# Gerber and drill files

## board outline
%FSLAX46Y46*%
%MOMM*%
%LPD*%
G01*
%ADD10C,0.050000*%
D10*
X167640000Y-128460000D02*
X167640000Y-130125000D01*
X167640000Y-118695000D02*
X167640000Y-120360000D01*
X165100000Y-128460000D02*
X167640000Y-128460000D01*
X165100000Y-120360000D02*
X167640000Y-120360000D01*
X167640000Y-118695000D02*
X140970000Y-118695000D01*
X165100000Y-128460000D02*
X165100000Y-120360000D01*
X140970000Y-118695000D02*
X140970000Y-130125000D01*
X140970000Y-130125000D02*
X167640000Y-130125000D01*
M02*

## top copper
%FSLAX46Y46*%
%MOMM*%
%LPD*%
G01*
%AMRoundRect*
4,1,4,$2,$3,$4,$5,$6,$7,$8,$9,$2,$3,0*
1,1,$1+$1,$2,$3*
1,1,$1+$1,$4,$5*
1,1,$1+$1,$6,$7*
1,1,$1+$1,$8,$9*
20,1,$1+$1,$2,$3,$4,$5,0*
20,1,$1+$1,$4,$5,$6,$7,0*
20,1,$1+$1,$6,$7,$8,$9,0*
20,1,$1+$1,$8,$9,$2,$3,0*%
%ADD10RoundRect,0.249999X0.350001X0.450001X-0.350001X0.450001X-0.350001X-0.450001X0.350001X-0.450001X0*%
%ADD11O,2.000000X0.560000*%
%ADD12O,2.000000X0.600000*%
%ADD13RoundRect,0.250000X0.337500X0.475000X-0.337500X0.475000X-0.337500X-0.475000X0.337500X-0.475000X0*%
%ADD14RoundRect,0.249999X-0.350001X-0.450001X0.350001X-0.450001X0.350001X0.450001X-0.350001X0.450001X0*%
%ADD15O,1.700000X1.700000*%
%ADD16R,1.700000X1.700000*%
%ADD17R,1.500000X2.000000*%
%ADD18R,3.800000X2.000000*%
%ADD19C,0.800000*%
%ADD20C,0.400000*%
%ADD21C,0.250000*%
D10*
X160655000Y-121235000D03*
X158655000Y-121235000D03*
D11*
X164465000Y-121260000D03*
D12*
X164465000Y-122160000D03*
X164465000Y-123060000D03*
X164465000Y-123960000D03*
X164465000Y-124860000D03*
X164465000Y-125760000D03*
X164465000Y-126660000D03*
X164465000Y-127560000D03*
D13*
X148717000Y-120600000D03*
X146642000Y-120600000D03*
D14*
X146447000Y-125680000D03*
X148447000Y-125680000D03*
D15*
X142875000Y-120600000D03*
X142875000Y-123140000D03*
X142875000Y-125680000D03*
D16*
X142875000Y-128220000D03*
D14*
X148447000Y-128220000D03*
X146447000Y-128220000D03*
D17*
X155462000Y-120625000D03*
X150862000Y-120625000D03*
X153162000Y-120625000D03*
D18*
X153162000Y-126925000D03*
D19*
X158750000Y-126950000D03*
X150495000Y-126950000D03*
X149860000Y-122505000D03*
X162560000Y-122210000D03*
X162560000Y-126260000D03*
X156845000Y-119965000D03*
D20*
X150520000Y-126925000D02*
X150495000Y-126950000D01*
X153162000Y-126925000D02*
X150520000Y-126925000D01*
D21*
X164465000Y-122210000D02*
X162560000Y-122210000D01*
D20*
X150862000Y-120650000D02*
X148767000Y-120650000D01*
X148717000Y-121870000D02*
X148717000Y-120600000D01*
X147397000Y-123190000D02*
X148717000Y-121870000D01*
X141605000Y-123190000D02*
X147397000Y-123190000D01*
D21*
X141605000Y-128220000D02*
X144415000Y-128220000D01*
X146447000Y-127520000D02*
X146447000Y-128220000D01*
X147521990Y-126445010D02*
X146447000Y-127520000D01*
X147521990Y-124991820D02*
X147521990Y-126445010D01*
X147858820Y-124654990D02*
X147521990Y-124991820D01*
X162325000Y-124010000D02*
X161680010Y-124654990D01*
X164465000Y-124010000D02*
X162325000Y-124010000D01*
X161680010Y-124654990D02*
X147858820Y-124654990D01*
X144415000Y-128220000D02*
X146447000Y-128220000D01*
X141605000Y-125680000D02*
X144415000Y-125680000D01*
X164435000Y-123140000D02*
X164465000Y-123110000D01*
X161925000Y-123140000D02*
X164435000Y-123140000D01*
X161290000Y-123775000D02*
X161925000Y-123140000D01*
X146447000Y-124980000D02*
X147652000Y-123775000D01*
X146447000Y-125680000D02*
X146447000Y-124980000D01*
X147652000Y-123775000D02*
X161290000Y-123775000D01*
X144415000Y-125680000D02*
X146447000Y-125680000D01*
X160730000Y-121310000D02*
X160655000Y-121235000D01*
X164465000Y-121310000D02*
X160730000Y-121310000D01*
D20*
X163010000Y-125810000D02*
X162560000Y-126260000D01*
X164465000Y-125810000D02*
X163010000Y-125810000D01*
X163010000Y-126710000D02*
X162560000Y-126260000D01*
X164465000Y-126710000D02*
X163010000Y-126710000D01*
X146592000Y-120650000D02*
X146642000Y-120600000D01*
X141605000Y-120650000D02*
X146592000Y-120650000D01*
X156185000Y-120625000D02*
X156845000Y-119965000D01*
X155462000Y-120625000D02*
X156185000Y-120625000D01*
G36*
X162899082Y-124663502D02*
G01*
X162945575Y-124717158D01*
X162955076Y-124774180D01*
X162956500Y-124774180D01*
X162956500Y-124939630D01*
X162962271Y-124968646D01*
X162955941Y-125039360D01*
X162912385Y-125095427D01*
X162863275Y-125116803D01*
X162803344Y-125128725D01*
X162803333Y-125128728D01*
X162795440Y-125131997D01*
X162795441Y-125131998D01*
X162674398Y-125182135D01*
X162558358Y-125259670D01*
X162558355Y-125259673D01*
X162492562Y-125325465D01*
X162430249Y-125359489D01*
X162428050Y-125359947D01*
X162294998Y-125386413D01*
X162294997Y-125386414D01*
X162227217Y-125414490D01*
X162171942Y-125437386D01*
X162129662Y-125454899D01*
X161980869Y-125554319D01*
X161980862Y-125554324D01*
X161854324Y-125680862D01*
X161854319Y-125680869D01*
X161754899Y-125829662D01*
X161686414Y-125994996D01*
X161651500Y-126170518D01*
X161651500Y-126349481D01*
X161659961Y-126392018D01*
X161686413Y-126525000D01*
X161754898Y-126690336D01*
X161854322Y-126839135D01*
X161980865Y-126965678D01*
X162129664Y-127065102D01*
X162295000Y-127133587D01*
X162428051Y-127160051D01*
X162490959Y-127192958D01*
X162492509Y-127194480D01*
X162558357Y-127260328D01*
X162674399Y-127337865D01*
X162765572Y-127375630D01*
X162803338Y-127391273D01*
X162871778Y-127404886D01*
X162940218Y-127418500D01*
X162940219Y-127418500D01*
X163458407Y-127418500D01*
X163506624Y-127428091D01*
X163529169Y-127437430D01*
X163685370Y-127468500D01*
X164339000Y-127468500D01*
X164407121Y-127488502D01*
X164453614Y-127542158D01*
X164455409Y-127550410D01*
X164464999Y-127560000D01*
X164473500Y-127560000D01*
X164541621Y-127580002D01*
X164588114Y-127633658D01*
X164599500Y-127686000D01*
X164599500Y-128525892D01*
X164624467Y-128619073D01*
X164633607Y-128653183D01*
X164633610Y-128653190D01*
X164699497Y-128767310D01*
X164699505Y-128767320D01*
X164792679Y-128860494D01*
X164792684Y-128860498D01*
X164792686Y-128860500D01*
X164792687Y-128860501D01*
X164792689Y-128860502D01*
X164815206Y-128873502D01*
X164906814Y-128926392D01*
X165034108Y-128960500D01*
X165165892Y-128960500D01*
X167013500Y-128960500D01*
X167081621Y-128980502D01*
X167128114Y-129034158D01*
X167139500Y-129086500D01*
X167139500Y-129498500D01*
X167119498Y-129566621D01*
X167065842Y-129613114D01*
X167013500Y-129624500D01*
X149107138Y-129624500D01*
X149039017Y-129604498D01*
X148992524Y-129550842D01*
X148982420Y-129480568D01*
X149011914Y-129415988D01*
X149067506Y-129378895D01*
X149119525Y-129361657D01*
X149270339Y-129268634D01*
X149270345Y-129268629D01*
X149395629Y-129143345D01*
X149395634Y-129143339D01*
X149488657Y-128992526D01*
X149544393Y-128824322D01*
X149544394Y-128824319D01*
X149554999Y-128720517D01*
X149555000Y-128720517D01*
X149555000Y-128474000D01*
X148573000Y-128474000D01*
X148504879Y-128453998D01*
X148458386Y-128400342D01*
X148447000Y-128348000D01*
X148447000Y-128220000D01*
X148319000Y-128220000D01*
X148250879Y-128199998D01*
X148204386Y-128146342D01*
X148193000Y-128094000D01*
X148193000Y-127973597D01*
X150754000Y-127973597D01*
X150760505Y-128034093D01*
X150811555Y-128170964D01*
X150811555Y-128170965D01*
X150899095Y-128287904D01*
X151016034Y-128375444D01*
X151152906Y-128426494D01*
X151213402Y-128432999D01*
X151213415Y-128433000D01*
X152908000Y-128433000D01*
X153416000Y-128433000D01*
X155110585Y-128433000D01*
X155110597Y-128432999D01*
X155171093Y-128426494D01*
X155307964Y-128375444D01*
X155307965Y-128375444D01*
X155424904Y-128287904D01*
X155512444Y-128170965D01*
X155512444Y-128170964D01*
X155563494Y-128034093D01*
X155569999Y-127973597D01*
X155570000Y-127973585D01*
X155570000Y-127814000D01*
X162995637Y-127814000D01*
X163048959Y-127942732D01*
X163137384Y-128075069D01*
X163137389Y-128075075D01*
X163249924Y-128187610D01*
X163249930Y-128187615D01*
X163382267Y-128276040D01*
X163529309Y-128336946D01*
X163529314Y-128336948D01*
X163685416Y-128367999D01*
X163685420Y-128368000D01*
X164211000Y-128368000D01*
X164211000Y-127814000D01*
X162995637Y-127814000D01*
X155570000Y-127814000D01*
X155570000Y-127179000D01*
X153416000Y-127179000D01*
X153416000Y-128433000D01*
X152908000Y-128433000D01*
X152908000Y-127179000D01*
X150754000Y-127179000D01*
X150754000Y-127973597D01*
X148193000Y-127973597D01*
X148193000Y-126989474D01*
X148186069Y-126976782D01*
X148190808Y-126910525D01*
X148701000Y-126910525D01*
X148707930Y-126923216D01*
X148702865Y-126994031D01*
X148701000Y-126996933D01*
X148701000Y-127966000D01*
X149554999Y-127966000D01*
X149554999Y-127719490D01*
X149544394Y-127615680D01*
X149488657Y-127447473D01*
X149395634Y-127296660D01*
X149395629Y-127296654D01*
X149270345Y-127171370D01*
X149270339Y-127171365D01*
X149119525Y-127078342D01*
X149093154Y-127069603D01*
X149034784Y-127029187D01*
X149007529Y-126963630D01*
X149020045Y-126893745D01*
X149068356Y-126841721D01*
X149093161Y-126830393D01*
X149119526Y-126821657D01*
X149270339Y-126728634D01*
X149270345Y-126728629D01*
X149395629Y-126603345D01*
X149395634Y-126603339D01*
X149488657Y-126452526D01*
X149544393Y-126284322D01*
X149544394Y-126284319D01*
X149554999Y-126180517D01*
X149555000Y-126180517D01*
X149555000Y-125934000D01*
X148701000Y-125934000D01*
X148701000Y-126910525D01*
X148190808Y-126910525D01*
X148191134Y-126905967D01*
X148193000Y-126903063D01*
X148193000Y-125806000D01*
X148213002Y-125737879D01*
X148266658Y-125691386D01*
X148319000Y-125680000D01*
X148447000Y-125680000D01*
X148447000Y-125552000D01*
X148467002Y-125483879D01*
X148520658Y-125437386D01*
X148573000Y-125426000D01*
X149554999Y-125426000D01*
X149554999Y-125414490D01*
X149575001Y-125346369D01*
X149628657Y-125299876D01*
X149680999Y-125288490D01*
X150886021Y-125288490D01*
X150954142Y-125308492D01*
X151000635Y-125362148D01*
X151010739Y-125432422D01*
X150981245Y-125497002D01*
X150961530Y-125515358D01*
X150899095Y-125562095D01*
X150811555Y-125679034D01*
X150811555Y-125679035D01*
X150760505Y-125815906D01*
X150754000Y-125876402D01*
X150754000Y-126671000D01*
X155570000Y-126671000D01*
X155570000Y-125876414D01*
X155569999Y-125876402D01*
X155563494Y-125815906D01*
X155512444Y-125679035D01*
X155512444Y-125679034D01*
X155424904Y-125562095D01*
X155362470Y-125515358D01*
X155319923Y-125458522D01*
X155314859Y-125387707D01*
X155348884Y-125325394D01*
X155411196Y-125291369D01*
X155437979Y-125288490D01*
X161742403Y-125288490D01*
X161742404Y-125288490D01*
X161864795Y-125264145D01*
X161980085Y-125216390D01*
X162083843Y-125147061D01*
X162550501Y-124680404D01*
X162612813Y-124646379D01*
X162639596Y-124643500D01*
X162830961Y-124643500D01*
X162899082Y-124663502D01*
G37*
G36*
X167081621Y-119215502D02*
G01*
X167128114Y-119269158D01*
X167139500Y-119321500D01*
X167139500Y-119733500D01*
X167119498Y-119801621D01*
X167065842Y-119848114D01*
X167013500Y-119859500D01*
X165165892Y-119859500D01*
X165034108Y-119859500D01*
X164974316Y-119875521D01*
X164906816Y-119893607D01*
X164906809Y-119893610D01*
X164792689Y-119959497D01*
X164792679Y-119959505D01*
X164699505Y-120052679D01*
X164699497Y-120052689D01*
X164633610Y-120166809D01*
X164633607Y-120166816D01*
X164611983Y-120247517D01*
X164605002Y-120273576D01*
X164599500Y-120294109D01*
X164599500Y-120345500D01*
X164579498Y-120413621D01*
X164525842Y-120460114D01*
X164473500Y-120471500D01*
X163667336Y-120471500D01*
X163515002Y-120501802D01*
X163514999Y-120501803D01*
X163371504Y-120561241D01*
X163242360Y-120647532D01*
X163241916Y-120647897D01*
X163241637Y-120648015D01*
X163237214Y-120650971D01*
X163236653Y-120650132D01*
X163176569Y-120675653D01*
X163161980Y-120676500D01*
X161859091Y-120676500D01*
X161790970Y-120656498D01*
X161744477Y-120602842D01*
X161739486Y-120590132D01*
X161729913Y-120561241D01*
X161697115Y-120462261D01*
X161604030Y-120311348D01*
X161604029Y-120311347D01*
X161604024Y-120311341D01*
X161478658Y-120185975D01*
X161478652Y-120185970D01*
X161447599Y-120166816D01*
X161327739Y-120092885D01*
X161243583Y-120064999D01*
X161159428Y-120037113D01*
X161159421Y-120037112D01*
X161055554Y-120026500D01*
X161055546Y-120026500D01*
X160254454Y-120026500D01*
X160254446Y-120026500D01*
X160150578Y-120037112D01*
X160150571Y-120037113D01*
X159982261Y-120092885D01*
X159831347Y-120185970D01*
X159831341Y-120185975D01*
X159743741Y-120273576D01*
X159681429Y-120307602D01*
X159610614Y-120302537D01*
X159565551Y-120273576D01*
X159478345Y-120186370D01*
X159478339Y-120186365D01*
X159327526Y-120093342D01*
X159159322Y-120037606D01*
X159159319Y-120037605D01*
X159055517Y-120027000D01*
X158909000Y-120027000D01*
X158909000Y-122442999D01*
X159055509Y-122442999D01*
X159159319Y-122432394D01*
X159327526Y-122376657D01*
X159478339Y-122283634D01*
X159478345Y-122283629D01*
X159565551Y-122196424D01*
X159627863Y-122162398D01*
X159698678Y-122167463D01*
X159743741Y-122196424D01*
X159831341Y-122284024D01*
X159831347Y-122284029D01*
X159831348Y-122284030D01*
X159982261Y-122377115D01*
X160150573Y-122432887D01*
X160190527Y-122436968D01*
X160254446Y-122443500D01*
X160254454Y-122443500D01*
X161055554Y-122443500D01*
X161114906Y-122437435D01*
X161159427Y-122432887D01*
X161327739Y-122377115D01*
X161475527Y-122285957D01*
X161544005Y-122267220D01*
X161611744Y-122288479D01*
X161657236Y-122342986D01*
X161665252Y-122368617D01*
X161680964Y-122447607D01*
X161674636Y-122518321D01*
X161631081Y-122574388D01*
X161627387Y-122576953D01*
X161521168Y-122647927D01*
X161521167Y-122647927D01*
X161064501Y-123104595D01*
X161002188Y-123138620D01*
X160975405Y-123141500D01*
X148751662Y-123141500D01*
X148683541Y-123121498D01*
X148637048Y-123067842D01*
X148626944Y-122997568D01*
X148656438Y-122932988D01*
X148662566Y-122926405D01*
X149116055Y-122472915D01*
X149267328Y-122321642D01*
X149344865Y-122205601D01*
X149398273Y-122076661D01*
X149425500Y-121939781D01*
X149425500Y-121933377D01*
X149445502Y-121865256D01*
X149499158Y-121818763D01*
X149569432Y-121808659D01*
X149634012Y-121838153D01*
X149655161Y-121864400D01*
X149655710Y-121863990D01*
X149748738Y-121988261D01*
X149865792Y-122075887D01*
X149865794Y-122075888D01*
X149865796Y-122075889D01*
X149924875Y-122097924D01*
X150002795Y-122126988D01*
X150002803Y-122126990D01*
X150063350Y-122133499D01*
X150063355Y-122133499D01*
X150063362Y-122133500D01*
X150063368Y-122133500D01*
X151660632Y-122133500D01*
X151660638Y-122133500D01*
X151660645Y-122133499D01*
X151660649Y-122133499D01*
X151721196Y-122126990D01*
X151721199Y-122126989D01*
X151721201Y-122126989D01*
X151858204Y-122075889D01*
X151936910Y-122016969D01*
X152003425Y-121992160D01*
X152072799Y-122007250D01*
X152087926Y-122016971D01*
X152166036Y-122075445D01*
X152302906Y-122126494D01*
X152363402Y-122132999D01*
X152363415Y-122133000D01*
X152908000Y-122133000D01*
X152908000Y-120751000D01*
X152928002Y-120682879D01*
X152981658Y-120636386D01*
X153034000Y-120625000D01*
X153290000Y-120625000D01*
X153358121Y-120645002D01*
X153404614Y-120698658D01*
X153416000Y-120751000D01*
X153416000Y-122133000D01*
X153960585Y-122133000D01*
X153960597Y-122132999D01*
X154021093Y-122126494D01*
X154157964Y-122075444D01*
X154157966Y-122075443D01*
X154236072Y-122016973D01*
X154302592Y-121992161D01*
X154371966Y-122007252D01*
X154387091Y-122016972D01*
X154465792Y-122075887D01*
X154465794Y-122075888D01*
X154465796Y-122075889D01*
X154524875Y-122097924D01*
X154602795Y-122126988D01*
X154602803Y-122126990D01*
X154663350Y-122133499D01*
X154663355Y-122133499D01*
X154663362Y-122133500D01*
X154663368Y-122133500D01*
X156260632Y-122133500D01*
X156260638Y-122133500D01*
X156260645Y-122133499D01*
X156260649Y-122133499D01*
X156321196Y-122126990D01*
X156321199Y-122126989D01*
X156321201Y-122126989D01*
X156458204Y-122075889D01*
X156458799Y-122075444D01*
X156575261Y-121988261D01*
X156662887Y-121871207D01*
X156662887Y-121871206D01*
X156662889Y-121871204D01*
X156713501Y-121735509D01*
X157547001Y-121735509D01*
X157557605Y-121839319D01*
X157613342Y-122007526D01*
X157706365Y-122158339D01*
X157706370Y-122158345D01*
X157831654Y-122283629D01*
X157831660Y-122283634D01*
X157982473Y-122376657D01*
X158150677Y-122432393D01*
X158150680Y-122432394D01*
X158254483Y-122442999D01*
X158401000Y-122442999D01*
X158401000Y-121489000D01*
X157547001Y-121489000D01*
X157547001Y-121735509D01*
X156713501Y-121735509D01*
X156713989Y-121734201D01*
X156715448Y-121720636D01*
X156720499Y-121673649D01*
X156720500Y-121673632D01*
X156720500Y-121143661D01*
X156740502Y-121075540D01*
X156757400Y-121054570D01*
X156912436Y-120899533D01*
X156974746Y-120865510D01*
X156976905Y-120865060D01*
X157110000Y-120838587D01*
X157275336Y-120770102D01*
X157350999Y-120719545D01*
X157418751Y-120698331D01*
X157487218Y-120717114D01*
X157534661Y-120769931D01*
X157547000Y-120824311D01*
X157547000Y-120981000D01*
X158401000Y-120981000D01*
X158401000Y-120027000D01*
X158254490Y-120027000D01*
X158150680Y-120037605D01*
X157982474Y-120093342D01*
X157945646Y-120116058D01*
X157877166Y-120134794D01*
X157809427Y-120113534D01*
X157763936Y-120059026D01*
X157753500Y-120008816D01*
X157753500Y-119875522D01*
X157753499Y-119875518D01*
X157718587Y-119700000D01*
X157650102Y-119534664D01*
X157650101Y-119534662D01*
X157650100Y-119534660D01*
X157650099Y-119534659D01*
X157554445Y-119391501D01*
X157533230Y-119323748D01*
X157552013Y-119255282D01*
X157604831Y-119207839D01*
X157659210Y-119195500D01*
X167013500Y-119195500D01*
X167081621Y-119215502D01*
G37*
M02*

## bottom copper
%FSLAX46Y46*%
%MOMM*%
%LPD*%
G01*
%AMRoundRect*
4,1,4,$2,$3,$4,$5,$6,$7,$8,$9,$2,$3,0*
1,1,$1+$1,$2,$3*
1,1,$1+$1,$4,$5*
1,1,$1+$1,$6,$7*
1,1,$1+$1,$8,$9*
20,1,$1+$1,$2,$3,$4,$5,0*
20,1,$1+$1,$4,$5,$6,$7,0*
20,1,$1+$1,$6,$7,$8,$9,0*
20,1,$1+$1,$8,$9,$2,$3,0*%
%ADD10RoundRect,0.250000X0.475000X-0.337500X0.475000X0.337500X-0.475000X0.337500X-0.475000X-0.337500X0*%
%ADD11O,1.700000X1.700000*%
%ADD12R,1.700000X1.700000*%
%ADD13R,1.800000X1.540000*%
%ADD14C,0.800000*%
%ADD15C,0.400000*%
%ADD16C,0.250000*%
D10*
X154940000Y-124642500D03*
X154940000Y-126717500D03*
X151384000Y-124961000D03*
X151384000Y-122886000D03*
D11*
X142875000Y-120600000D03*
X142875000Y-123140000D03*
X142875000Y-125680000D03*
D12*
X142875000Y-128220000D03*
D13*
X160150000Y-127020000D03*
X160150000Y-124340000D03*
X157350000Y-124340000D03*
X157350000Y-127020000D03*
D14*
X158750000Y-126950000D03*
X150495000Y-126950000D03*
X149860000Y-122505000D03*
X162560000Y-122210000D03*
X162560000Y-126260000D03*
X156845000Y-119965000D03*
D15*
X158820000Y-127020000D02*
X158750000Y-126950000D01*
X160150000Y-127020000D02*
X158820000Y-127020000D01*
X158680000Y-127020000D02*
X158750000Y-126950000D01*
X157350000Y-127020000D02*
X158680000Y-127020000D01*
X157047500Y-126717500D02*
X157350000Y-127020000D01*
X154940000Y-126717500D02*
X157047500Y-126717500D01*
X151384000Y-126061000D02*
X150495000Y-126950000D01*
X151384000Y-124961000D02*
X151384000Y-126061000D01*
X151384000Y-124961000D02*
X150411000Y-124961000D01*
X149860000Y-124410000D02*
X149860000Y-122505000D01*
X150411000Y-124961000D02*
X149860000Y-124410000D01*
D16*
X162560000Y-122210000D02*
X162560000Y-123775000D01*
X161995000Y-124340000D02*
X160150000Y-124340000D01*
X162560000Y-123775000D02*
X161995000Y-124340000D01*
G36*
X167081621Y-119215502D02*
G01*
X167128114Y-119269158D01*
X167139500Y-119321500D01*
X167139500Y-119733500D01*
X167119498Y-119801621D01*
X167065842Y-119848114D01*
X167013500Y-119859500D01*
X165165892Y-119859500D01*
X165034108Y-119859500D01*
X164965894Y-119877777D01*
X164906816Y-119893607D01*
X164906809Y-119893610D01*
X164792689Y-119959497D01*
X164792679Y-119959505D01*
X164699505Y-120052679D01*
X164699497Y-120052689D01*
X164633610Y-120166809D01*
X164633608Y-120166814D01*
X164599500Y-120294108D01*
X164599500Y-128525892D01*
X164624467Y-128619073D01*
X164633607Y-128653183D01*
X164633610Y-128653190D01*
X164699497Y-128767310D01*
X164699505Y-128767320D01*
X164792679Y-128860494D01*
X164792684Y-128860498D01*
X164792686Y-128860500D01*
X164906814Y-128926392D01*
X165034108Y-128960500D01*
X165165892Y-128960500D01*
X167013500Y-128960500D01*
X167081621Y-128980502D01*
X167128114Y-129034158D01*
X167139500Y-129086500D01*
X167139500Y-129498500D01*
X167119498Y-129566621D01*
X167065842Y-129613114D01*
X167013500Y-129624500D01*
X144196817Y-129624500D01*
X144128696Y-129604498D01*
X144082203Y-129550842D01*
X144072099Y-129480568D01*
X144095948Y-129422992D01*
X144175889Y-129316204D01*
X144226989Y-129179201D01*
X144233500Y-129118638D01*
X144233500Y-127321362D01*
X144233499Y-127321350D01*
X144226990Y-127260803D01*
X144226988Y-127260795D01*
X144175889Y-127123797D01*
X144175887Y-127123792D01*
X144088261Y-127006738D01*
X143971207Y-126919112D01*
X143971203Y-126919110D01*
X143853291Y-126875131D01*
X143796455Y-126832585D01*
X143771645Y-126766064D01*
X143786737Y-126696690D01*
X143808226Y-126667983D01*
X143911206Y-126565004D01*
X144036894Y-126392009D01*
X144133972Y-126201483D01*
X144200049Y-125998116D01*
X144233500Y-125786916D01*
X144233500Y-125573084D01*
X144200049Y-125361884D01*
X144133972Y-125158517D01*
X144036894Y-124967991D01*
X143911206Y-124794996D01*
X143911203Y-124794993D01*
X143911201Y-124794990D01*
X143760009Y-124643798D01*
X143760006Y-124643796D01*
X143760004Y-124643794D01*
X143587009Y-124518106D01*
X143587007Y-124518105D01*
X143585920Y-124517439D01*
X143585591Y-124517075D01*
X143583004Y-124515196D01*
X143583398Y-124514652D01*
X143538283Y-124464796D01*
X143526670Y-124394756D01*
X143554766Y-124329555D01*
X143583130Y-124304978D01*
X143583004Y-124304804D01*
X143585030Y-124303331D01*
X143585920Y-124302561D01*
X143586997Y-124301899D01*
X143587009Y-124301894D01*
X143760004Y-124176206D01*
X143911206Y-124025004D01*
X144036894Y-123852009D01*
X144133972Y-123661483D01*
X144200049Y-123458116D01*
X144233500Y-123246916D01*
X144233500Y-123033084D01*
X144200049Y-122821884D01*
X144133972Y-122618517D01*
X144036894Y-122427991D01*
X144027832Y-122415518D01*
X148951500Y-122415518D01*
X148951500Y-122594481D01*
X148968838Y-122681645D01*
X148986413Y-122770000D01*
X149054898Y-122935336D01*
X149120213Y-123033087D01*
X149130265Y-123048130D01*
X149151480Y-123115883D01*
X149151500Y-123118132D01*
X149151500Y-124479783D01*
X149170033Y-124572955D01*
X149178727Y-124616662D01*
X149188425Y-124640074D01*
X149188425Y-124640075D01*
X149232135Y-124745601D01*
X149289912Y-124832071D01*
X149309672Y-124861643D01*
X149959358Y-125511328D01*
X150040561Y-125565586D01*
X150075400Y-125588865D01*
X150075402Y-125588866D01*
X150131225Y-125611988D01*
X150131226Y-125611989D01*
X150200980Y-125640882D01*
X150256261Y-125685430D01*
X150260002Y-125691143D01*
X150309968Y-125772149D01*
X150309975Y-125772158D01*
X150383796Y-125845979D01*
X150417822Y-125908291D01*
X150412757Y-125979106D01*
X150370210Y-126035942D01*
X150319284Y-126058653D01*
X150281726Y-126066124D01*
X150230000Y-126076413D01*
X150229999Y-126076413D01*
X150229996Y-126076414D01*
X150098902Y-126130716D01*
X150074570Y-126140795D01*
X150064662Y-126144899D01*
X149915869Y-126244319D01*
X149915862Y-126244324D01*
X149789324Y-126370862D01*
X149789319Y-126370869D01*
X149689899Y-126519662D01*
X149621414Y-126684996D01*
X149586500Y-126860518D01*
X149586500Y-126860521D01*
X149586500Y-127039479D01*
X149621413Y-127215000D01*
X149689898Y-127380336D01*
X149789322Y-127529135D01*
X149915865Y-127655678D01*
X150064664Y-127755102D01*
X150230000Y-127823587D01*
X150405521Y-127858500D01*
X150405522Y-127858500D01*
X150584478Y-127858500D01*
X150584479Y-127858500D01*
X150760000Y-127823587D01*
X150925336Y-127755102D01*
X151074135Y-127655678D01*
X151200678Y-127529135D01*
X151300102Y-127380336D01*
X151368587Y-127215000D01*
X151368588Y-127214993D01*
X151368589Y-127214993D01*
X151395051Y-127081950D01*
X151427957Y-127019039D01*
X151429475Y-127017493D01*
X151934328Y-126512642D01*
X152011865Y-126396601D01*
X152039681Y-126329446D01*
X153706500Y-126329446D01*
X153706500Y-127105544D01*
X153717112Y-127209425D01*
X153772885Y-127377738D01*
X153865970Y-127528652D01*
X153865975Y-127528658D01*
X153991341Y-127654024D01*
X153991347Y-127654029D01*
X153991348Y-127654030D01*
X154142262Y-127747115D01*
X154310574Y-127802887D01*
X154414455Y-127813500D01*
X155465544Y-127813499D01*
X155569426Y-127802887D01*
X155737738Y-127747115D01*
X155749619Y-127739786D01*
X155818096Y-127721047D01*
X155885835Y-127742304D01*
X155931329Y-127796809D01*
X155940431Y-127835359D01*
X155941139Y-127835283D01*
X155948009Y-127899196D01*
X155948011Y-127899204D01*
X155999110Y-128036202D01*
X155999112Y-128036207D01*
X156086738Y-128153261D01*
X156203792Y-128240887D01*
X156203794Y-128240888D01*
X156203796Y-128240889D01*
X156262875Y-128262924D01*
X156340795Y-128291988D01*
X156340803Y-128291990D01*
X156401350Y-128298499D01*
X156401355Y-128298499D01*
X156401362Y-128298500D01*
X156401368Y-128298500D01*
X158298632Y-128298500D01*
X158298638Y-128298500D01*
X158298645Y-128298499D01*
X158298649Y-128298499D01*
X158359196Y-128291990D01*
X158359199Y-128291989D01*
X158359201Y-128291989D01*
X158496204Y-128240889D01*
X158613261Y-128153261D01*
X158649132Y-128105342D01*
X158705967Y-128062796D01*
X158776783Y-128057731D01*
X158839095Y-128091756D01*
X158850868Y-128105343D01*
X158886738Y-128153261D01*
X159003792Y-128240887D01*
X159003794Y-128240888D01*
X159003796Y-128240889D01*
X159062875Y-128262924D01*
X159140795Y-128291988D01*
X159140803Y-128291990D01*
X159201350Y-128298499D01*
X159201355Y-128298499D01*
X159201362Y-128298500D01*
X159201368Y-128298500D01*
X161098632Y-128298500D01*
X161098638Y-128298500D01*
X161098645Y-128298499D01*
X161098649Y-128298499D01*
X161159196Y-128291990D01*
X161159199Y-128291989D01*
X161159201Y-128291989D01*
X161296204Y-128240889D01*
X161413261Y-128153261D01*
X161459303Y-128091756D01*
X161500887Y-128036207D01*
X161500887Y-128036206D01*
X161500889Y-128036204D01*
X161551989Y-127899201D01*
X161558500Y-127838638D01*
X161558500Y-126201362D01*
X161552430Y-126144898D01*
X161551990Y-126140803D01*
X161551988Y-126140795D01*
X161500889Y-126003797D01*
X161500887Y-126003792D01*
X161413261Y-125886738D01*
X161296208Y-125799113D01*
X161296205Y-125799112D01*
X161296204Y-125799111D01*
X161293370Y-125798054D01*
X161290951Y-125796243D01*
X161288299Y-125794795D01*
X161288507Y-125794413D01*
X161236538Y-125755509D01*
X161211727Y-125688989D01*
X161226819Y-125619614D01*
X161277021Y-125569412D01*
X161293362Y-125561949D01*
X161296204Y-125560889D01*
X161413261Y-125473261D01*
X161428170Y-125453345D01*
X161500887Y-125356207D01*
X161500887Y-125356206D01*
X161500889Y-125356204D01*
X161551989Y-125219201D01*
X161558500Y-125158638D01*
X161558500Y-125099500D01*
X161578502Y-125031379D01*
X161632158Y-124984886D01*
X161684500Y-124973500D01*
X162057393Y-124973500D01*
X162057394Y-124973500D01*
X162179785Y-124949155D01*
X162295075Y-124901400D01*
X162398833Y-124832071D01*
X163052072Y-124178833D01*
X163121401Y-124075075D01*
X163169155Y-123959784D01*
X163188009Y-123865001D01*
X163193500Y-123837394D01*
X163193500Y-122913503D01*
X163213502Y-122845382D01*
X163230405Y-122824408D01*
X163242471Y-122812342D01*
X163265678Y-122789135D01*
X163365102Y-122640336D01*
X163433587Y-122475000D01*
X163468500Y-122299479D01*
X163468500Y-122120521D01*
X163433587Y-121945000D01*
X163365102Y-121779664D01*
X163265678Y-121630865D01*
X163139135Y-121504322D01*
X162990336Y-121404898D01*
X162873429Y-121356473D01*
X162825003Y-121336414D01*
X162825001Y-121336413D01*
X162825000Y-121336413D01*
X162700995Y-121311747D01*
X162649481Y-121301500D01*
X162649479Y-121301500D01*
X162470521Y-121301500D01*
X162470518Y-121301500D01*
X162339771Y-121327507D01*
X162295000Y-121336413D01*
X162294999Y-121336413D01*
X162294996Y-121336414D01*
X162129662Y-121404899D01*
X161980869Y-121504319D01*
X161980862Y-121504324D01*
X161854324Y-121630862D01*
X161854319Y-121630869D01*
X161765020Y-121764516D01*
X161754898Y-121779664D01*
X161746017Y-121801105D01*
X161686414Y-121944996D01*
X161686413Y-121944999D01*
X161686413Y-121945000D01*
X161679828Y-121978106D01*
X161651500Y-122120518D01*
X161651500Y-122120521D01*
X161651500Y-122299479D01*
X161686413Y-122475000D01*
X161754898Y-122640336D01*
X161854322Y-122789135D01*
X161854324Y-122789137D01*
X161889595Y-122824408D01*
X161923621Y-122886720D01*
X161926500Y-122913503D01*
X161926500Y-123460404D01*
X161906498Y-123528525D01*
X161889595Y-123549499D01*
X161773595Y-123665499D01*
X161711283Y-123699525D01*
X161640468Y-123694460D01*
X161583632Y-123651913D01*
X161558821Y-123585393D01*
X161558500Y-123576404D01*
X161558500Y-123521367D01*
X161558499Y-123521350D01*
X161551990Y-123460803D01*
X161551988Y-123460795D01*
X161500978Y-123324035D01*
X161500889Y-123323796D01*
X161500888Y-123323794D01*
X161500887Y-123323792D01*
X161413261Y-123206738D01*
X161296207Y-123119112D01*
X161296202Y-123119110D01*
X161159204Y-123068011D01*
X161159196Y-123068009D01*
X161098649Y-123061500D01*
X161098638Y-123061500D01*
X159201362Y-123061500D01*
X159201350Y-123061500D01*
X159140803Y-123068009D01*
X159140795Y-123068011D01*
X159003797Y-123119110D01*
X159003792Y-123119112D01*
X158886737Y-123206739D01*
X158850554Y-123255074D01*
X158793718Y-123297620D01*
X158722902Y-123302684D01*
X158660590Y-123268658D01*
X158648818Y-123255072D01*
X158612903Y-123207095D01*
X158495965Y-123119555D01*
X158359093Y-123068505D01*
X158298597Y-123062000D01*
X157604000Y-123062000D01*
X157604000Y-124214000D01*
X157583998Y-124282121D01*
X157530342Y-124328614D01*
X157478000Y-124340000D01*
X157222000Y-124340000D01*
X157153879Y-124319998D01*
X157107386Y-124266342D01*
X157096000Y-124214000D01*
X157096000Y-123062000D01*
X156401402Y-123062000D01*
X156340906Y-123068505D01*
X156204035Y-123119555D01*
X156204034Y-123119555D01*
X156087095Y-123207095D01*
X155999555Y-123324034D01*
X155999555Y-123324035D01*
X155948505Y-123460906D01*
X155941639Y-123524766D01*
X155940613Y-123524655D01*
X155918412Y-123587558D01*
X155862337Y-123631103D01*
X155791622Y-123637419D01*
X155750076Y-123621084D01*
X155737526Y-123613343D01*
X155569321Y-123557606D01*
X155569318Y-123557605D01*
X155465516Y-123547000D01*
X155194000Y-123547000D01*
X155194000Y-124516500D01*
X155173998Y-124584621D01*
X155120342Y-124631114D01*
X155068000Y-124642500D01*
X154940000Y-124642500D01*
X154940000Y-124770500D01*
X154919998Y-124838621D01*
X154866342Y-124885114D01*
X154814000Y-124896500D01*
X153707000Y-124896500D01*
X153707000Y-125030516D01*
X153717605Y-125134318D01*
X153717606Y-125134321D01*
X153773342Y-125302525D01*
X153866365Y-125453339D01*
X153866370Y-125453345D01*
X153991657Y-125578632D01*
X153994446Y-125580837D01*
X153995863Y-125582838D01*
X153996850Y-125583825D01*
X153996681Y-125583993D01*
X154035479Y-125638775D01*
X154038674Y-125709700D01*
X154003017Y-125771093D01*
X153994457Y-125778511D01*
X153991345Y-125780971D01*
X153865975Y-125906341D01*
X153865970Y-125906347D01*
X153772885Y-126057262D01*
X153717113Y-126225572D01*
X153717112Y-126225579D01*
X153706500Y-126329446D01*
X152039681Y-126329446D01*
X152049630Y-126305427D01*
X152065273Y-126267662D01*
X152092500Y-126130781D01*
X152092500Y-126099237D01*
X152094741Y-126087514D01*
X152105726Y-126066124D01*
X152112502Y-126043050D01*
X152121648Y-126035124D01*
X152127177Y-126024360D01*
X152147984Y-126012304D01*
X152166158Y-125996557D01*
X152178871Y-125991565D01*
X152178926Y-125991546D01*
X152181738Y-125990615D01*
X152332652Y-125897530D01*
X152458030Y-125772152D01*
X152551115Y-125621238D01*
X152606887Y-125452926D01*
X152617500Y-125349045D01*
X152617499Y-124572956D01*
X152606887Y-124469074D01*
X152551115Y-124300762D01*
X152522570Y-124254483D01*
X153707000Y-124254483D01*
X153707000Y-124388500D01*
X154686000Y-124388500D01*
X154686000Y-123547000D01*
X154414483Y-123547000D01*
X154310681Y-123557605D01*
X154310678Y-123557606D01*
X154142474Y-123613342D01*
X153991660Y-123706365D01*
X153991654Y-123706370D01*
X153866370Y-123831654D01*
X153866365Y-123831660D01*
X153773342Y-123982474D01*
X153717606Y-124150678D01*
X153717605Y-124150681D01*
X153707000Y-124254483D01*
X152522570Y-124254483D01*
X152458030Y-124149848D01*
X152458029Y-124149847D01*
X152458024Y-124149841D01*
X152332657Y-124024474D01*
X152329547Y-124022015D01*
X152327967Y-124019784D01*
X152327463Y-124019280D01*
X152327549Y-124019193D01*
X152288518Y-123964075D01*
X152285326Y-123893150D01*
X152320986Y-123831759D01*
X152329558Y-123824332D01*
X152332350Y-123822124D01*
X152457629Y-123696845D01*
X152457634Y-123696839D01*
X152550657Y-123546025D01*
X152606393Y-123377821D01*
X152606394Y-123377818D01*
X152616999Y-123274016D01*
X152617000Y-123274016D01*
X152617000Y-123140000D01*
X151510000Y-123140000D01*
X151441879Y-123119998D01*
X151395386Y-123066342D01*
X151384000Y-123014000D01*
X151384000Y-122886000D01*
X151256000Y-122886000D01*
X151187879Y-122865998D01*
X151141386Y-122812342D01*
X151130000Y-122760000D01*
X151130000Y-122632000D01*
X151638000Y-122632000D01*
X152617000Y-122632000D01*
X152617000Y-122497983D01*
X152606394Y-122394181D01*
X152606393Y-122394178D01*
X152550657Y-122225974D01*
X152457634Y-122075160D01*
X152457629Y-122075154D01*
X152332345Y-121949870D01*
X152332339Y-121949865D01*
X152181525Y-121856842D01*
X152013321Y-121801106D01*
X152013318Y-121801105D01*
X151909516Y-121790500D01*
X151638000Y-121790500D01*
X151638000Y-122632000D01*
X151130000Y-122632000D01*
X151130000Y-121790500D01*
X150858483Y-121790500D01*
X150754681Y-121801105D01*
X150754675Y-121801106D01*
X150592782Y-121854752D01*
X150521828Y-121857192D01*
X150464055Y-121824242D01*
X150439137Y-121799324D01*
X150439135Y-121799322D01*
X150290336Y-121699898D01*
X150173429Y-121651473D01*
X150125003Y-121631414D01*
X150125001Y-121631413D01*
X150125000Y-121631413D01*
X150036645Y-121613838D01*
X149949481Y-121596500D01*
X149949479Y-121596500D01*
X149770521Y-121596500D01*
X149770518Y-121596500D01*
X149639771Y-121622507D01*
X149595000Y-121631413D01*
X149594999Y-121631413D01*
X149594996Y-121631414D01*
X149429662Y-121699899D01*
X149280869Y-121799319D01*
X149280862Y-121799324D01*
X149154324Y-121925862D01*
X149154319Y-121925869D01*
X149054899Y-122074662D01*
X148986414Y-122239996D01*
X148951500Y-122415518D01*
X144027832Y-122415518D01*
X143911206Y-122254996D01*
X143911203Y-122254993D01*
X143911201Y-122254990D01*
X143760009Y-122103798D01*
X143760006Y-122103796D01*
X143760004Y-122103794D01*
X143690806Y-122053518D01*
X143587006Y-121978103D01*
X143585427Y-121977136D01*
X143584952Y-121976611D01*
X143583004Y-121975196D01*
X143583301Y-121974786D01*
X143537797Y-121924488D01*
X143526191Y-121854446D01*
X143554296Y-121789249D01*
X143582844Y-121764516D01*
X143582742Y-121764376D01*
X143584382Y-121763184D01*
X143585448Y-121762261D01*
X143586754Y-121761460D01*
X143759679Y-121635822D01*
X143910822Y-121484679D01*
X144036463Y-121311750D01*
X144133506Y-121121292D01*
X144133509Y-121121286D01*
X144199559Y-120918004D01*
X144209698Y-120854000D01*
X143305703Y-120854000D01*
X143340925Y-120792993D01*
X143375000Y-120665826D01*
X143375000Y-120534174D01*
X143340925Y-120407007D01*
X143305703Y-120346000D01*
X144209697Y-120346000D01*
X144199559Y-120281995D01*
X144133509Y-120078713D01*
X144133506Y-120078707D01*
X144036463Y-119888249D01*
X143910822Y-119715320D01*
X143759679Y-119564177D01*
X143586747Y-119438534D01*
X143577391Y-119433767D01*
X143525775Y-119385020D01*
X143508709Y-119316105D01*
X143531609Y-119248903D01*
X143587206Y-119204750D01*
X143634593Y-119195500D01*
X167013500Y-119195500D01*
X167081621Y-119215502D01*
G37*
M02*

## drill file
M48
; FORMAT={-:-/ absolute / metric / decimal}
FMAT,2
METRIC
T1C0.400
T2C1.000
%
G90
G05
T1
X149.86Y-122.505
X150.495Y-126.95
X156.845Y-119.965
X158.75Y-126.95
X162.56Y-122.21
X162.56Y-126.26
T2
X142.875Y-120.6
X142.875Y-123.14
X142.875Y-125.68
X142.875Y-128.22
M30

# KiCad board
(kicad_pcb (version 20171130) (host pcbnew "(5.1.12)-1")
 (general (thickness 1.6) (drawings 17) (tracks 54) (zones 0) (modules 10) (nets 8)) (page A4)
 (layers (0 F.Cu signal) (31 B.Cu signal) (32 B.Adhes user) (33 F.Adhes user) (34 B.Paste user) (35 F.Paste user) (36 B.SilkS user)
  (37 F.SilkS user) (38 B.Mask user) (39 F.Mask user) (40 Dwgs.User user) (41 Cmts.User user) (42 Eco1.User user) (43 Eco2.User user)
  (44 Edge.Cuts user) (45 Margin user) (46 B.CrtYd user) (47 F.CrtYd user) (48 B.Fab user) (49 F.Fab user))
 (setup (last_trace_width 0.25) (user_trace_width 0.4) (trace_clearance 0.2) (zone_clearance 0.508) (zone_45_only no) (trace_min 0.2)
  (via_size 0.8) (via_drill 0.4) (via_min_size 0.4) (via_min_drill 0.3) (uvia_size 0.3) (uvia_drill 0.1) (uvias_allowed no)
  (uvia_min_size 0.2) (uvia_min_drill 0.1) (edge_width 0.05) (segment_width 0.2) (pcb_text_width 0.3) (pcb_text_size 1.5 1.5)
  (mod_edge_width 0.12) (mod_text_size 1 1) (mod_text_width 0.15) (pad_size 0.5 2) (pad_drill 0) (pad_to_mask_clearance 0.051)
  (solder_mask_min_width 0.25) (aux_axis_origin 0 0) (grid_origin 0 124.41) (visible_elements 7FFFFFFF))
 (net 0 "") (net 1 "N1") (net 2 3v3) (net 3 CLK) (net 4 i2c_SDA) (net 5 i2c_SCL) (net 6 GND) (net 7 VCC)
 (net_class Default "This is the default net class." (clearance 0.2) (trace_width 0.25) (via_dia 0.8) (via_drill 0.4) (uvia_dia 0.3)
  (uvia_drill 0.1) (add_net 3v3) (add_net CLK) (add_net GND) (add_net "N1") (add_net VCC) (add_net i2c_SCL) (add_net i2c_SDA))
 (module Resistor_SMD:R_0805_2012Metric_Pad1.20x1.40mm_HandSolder (layer F.Cu) (at 159.655 121.235 180)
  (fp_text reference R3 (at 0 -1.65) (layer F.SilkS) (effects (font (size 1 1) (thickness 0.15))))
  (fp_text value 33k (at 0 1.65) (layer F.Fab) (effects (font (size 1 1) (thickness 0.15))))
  (pad 1 smd roundrect (at -1 0 180) (size 1.2 1.4) (layers F.Cu F.Paste F.Mask) (roundrect_rratio 0.2083325) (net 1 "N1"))
  (pad 2 smd roundrect (at 1 0 180) (size 1.2 1.4) (layers F.Cu F.Paste F.Mask) (roundrect_rratio 0.2083325) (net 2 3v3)))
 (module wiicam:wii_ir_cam (layer F.Cu) (at 164.465 124.41 90)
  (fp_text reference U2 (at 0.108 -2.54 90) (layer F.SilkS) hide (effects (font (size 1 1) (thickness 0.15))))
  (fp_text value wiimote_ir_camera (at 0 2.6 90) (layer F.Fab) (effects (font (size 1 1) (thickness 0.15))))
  (pad 8 smd oval (at 3.15 0 90) (size 0.56 2) (layers F.Cu F.Paste F.Mask) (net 1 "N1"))
  (pad 7 smd oval (at 2.25 0 90) (size 0.6 2) (layers F.Cu F.Paste F.Mask) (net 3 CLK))
  (pad 6 smd oval (at 1.35 0 90) (size 0.6 2) (layers F.Cu F.Paste F.Mask) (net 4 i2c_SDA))
  (pad 5 smd oval (at 0.45 0 90) (size 0.6 2) (layers F.Cu F.Paste F.Mask) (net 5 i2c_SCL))
  (pad 4 smd oval (at -0.45 0 90) (size 0.6 2) (layers F.Cu F.Paste F.Mask))
  (pad 3 smd oval (at -1.35 0 90) (size 0.6 2) (layers F.Cu F.Paste F.Mask) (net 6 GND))
  (pad 2 smd oval (at -2.25 0 90) (size 0.6 2) (layers F.Cu F.Paste F.Mask) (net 6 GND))
  (pad 1 smd oval (at -3.15 0 90) (size 0.6 2) (layers F.Cu F.Paste F.Mask) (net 2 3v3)))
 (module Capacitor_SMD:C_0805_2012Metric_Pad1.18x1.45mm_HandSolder (layer B.Cu) (at 154.94 125.68 90)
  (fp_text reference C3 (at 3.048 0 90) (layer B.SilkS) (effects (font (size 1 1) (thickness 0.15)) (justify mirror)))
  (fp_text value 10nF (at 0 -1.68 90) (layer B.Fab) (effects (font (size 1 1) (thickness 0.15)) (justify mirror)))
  (pad 2 smd roundrect (at 1.0375 0 90) (size 1.175 1.45) (layers B.Cu B.Paste B.Mask) (roundrect_rratio 0.2127659574468085) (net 6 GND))
  (pad 1 smd roundrect (at -1.0375 0 90) (size 1.175 1.45) (layers B.Cu B.Paste B.Mask) (roundrect_rratio 0.2127659574468085) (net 2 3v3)))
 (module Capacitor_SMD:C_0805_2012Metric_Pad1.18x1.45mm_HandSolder (layer F.Cu) (at 147.6795 120.6 180)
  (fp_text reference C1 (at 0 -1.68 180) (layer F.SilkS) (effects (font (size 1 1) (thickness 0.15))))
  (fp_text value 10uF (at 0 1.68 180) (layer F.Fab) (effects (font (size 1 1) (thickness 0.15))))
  (pad 1 smd roundrect (at -1.0375 0 180) (size 1.175 1.45) (layers F.Cu F.Paste F.Mask) (roundrect_rratio 0.2127659574468085) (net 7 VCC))
  (pad 2 smd roundrect (at 1.0375 0 180) (size 1.175 1.45) (layers F.Cu F.Paste F.Mask) (roundrect_rratio 0.2127659574468085) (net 6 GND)))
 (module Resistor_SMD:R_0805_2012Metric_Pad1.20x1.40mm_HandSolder (layer F.Cu) (at 147.447 125.68)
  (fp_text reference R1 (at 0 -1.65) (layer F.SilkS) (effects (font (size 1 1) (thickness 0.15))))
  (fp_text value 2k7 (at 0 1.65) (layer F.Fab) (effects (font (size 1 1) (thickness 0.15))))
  (pad 1 smd roundrect (at -1 0) (size 1.2 1.4) (layers F.Cu F.Paste F.Mask) (roundrect_rratio 0.2083325) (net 4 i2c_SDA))
  (pad 2 smd roundrect (at 1 0) (size 1.2 1.4) (layers F.Cu F.Paste F.Mask) (roundrect_rratio 0.2083325) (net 2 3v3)))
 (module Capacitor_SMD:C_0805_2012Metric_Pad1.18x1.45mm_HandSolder (layer B.Cu) (at 151.384 123.9235 90)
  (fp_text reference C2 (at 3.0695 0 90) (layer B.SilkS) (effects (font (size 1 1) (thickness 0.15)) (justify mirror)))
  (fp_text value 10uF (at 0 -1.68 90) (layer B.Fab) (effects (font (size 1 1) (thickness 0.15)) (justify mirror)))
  (pad 1 smd roundrect (at -1.0375 0 90) (size 1.175 1.45) (layers B.Cu B.Paste B.Mask) (roundrect_rratio 0.2127659574468085) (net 2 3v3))
  (pad 2 smd roundrect (at 1.0375 0 90) (size 1.175 1.45) (layers B.Cu B.Paste B.Mask) (roundrect_rratio 0.2127659574468085) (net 6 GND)))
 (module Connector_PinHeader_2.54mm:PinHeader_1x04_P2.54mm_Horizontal (layer F.Cu) (at 142.875 128.22 180)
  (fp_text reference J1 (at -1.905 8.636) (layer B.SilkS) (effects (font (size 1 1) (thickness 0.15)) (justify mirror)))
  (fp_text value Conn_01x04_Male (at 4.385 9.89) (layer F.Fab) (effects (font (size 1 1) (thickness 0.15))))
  (pad 4 thru_hole oval (at 0 7.62 180) (size 1.7 1.7) (drill 1) (layers *.Cu *.Mask) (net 6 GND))
  (pad 3 thru_hole oval (at 0 5.08 180) (size 1.7 1.7) (drill 1) (layers *.Cu *.Mask) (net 7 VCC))
  (pad 2 thru_hole oval (at 0 2.54 180) (size 1.7 1.7) (drill 1) (layers *.Cu *.Mask) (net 4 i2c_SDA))
  (pad 1 thru_hole rect (at 0 0 180) (size 1.7 1.7) (drill 1) (layers *.Cu *.Mask) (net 5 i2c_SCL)))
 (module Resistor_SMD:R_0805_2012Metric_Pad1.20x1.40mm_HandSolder (layer F.Cu) (at 147.447 128.22)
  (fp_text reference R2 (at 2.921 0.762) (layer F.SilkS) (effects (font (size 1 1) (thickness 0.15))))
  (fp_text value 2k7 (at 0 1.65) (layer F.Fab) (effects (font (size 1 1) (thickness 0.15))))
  (pad 2 smd roundrect (at 1 0) (size 1.2 1.4) (layers F.Cu F.Paste F.Mask) (roundrect_rratio 0.2083325) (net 2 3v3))
  (pad 1 smd roundrect (at -1 0) (size 1.2 1.4) (layers F.Cu F.Paste F.Mask) (roundrect_rratio 0.2083325) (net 5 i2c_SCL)))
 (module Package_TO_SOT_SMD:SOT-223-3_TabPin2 (layer F.Cu) (at 153.162 123.775 270)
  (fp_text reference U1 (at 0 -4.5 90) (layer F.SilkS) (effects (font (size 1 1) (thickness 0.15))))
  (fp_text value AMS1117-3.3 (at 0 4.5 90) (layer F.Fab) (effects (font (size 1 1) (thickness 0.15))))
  (pad 1 smd rect (at -3.15 -2.3 270) (size 2 1.5) (layers F.Cu F.Paste F.Mask) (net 6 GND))
  (pad 3 smd rect (at -3.15 2.3 270) (size 2 1.5) (layers F.Cu F.Paste F.Mask) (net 7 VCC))
  (pad 2 smd rect (at -3.15 0 270) (size 2 1.5) (layers F.Cu F.Paste F.Mask) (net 2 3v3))
  (pad 2 smd rect (at 3.15 0 270) (size 2 3.8) (layers F.Cu F.Paste F.Mask) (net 2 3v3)))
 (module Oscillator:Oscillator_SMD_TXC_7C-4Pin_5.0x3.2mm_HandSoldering (layer B.Cu) (at 158.75 125.68 90)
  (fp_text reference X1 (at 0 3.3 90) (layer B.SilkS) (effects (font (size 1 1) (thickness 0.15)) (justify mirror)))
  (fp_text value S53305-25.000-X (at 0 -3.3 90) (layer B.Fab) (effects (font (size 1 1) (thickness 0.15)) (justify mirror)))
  (pad 4 smd rect (at -1.34 1.4 90) (size 1.54 1.8) (layers B.Cu B.Paste B.Mask) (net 2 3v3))
  (pad 3 smd rect (at 1.34 1.4 90) (size 1.54 1.8) (layers B.Cu B.Paste B.Mask) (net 3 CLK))
  (pad 2 smd rect (at 1.34 -1.4 90) (size 1.54 1.8) (layers B.Cu B.Paste B.Mask) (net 6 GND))
  (pad 1 smd rect (at -1.34 -1.4 90) (size 1.54 1.8) (layers B.Cu B.Paste B.Mask) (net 2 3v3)))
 (gr_line (start 167.64 128.46) (end 167.64 130.125) (layer Edge.Cuts) (width 0.05))
 (gr_line (start 167.64 118.695) (end 167.64 120.36) (layer Edge.Cuts) (width 0.05))
 (gr_line (start 165.1 128.46) (end 167.64 128.46) (layer Edge.Cuts) (width 0.05))
 (gr_line (start 165.1 120.36) (end 167.64 120.36) (layer Edge.Cuts) (width 0.05))
 (gr_line (start 167.64 118.695) (end 140.97 118.695) (layer Edge.Cuts) (width 0.05))
 (gr_line (start 165.1 128.46) (end 165.1 120.36) (layer Edge.Cuts) (width 0.05))
 (gr_line (start 140.97 118.695) (end 140.97 130.125) (layer Edge.Cuts) (width 0.05))
 (gr_line (start 140.97 130.125) (end 167.64 130.125) (layer Edge.Cuts) (width 0.05))
 (via (at 158.75 126.95) (size 0.8) (drill 0.4) (layers F.Cu B.Cu) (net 2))
 (segment (start 158.82 127.02) (end 158.75 126.95) (width 0.4) (layer B.Cu) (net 2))
 (segment (start 160.15 127.02) (end 158.82 127.02) (width 0.4) (layer B.Cu) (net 2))
 (segment (start 158.68 127.02) (end 158.75 126.95) (width 0.4) (layer B.Cu) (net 2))
 (segment (start 157.35 127.02) (end 158.68 127.02) (width 0.4) (layer B.Cu) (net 2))
 (segment (start 157.0475 126.7175) (end 157.35 127.02) (width 0.4) (layer B.Cu) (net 2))
 (segment (start 154.94 126.7175) (end 157.0475 126.7175) (width 0.4) (layer B.Cu) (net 2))
 (via (at 150.495 126.95) (size 0.8) (drill 0.4) (layers F.Cu B.Cu) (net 2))
 (segment (start 150.52 126.925) (end 150.495 126.95) (width 0.4) (layer F.Cu) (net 2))
 (segment (start 153.162 126.925) (end 150.52 126.925) (width 0.4) (layer F.Cu) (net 2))
 (segment (start 151.384 126.061) (end 150.495 126.95) (width 0.4) (layer B.Cu) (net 2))
 (segment (start 151.384 124.961) (end 151.384 126.061) (width 0.4) (layer B.Cu) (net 2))
 (segment (start 151.384 124.961) (end 150.411 124.961) (width 0.4) (layer B.Cu) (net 2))
 (via (at 149.86 122.505) (size 0.8) (drill 0.4) (layers F.Cu B.Cu) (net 2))
 (segment (start 149.86 124.41) (end 149.86 122.505) (width 0.4) (layer B.Cu) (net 2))
 (segment (start 150.411 124.961) (end 149.86 124.41) (width 0.4) (layer B.Cu) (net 2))
 (via (at 162.56 122.21) (size 0.8) (drill 0.4) (layers F.Cu B.Cu) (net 3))
 (segment (start 164.465 122.21) (end 162.56 122.21) (width 0.25) (layer F.Cu) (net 3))
 (segment (start 162.56 122.21) (end 162.56 123.775) (width 0.25) (layer B.Cu) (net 3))
 (segment (start 161.995 124.34) (end 160.15 124.34) (width 0.25) (layer B.Cu) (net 3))
 (segment (start 162.56 123.775) (end 161.995 124.34) (width 0.25) (layer B.Cu) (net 3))
 (segment (start 150.862 120.65) (end 148.767 120.65) (width 0.4) (layer F.Cu) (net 7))
 (segment (start 148.717 121.87) (end 148.717 120.6) (width 0.4) (layer F.Cu) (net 7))
 (segment (start 147.397 123.19) (end 148.717 121.87) (width 0.4) (layer F.Cu) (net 7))
 (segment (start 141.605 123.19) (end 147.397 123.19) (width 0.4) (layer F.Cu) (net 7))
 (segment (start 141.605 128.22) (end 144.415 128.22) (width 0.25) (layer F.Cu) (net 5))
 (segment (start 146.447 127.52) (end 146.447 128.22) (width 0.25) (layer F.Cu) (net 5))
 (segment (start 147.52199 126.44501) (end 146.447 127.52) (width 0.25) (layer F.Cu) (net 5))
 (segment (start 147.52199 124.99182) (end 147.52199 126.44501) (width 0.25) (layer F.Cu) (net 5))
 (segment (start 147.85882 124.65499) (end 147.52199 124.99182) (width 0.25) (layer F.Cu) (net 5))
 (segment (start 162.325 124.01) (end 161.68001 124.65499) (width 0.25) (layer F.Cu) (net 5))
 (segment (start 164.465 124.01) (end 162.325 124.01) (width 0.25) (layer F.Cu) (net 5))
 (segment (start 161.68001 124.65499) (end 147.85882 124.65499) (width 0.25) (layer F.Cu) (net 5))
 (segment (start 144.415 128.22) (end 146.447 128.22) (width 0.25) (layer F.Cu) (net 5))
 (segment (start 141.605 125.68) (end 144.415 125.68) (width 0.25) (layer F.Cu) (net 4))
 (segment (start 164.435 123.14) (end 164.465 123.11) (width 0.25) (layer F.Cu) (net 4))
 (segment (start 161.925 123.14) (end 164.435 123.14) (width 0.25) (layer F.Cu) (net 4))
 (segment (start 161.29 123.775) (end 161.925 123.14) (width 0.25) (layer F.Cu) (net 4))
 (segment (start 146.447 124.98) (end 147.652 123.775) (width 0.25) (layer F.Cu) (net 4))
 (segment (start 146.447 125.68) (end 146.447 124.98) (width 0.25) (layer F.Cu) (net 4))
 (segment (start 147.652 123.775) (end 161.29 123.775) (width 0.25) (layer F.Cu) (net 4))
 (segment (start 144.415 125.68) (end 146.447 125.68) (width 0.25) (layer F.Cu) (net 4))
 (segment (start 160.73 121.31) (end 160.655 121.235) (width 0.25) (layer F.Cu) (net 1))
 (segment (start 164.465 121.31) (end 160.73 121.31) (width 0.25) (layer F.Cu) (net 1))
 (via (at 162.56 126.26) (size 0.8) (drill 0.4) (layers F.Cu B.Cu) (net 6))
 (segment (start 163.01 125.81) (end 162.56 126.26) (width 0.4) (layer F.Cu) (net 6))
 (segment (start 164.465 125.81) (end 163.01 125.81) (width 0.4) (layer F.Cu) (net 6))
 (segment (start 163.01 126.71) (end 162.56 126.26) (width 0.4) (layer F.Cu) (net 6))
 (segment (start 164.465 126.71) (end 163.01 126.71) (width 0.4) (layer F.Cu) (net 6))
 (segment (start 146.592 120.65) (end 146.642 120.6) (width 0.4) (layer F.Cu) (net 6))
 (segment (start 141.605 120.65) (end 146.592 120.65) (width 0.4) (layer F.Cu) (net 6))
 (via (at 156.845 119.965) (size 0.8) (drill 0.4) (layers F.Cu B.Cu) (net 6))
 (segment (start 156.185 120.625) (end 156.845 119.965) (width 0.4) (layer F.Cu) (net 6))
 (segment (start 155.462 120.625) (end 156.185 120.625) (width 0.4) (layer F.Cu) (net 6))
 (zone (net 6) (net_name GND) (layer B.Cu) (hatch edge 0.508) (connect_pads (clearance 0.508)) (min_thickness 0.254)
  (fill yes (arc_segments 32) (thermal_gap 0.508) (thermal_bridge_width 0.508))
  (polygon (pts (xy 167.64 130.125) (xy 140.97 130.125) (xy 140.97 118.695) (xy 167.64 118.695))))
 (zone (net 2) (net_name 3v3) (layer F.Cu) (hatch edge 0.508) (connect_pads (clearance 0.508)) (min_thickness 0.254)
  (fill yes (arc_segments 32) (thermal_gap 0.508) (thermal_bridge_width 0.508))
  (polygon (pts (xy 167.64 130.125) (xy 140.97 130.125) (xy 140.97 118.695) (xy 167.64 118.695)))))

